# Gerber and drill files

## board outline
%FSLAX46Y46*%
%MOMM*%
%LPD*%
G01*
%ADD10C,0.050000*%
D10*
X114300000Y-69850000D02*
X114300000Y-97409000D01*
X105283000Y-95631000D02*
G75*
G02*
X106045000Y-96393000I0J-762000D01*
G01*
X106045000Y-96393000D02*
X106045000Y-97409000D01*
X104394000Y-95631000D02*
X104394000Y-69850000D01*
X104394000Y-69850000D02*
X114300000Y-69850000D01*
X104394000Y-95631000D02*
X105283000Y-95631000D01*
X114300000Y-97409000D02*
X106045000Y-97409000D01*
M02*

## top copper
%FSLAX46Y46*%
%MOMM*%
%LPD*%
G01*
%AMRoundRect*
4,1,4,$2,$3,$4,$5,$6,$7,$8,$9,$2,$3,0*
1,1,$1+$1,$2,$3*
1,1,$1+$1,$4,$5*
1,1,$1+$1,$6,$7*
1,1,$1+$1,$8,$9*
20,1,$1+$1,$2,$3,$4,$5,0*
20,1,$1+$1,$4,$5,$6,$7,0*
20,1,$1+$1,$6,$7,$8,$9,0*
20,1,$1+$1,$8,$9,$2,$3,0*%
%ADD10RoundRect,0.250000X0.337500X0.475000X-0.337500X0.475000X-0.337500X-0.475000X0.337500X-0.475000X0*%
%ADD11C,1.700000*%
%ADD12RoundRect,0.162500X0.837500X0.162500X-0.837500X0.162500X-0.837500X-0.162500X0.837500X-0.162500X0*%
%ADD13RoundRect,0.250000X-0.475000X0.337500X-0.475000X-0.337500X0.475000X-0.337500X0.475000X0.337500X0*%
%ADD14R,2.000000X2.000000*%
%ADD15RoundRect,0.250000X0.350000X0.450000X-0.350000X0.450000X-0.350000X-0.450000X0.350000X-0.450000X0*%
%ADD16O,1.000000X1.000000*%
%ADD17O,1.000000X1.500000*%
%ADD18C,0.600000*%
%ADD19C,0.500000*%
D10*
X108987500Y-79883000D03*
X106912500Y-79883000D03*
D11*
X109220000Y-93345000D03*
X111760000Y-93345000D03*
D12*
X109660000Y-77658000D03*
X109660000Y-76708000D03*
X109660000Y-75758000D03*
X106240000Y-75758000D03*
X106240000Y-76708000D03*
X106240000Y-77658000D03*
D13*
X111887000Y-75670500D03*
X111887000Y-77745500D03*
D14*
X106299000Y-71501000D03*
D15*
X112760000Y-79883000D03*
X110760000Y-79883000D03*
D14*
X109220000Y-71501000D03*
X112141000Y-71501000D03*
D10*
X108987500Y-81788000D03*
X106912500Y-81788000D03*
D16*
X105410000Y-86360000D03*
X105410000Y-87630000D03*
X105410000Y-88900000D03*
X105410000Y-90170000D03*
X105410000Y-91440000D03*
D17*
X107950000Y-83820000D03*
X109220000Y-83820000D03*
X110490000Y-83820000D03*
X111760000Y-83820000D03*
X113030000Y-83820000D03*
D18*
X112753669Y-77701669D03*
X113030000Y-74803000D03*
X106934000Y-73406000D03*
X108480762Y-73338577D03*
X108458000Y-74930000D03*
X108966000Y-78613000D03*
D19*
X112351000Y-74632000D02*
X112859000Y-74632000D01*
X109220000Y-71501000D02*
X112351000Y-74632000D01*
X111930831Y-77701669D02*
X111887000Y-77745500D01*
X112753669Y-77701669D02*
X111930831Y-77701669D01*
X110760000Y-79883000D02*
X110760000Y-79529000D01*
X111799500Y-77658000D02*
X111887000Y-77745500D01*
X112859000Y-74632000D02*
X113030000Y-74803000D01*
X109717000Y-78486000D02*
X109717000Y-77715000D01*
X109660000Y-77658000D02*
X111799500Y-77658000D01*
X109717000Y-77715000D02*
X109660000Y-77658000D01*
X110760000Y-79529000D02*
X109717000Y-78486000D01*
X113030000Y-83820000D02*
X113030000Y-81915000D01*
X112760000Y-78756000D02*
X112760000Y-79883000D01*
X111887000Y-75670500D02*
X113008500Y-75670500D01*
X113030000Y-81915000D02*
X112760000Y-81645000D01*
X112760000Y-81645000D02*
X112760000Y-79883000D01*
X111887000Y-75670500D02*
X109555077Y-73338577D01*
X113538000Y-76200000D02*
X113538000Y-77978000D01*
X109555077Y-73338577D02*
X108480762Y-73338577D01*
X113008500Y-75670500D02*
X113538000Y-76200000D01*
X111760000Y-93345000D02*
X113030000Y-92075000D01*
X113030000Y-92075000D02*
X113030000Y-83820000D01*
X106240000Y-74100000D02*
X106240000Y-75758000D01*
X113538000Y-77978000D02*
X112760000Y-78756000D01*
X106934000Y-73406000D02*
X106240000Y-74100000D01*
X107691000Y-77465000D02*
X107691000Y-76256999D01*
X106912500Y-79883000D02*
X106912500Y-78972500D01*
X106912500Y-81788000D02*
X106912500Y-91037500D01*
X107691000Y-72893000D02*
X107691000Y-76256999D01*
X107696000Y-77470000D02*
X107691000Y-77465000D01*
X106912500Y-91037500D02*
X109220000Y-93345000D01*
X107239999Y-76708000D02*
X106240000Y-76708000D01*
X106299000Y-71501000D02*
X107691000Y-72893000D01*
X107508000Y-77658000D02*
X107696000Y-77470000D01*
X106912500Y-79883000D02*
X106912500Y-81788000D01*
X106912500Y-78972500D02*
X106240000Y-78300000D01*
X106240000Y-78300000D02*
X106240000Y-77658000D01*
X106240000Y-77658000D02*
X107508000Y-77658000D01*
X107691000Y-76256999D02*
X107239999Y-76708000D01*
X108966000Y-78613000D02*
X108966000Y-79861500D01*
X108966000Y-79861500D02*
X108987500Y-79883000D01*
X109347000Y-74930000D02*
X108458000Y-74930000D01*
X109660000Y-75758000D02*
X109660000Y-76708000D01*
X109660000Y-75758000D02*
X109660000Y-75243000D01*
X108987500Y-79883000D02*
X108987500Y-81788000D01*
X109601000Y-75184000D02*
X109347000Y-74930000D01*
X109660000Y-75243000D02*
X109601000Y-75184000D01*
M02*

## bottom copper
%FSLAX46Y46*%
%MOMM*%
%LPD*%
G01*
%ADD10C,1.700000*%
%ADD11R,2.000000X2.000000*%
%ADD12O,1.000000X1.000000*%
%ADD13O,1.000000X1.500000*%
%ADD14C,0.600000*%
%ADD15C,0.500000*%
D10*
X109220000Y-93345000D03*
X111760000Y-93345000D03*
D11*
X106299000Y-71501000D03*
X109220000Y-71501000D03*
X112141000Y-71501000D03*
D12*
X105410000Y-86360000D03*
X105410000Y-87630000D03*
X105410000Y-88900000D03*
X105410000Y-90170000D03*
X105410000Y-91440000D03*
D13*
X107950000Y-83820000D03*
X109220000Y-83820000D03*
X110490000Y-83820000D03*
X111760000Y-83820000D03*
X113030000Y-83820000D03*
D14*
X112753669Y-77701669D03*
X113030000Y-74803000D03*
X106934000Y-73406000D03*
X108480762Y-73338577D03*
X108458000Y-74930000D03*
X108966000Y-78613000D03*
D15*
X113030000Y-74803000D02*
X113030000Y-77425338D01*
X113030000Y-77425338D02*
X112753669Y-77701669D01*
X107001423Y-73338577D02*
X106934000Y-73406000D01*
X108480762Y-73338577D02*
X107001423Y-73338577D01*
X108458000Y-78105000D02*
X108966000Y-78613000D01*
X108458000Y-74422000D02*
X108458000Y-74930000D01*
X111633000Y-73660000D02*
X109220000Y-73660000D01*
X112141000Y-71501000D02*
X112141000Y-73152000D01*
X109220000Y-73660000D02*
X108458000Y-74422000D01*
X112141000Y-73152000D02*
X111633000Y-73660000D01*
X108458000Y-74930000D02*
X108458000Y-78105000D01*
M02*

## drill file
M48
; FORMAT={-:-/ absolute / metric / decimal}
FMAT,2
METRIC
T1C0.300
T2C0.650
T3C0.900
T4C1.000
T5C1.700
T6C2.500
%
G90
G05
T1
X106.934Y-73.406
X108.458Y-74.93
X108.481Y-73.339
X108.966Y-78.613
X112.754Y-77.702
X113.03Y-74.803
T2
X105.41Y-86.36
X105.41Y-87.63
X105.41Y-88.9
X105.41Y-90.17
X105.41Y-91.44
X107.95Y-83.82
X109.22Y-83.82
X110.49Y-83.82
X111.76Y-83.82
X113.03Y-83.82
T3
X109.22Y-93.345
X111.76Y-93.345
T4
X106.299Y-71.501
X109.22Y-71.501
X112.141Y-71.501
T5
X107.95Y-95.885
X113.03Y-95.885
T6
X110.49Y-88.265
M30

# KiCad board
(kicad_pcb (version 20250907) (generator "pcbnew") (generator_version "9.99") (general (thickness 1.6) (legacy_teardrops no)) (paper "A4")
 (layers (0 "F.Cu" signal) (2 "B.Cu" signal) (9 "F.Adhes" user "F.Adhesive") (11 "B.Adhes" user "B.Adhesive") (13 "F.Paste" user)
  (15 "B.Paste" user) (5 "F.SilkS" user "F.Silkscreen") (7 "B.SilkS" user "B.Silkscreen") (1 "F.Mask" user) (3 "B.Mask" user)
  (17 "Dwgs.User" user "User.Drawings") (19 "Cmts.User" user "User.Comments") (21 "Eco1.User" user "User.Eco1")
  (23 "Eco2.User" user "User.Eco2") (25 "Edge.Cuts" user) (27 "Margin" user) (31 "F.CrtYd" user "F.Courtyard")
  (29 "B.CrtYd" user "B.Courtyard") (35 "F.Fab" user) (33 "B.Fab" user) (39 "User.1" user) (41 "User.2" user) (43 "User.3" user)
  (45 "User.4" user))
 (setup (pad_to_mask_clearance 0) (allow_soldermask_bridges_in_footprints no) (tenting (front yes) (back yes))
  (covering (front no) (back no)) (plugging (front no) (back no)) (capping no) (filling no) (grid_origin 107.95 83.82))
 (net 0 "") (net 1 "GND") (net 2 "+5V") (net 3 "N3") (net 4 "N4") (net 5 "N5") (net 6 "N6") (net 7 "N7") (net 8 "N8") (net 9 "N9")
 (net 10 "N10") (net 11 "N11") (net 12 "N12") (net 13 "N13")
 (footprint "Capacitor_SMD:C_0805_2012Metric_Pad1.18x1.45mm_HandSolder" (layer "F.Cu") (at 107.95 79.883 180)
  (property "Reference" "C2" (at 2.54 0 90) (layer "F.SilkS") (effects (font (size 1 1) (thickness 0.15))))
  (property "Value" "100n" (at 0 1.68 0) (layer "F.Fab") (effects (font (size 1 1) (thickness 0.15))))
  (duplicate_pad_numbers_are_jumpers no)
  (pad "1" smd roundrect (at -1.0375 0 180) (size 1.175 1.45) (layers "F.Cu" "F.Mask" "F.Paste") (roundrect_rratio 0.212766) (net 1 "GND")
   (tenting (front none) (back none)))
  (pad "2" smd roundrect (at 1.0375 0 180) (size 1.175 1.45) (layers "F.Cu" "F.Mask" "F.Paste") (roundrect_rratio 0.212766) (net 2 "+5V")
   (tenting (front none) (back none))))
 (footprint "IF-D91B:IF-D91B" (layer "F.Cu") (at 110.49 88.265 180)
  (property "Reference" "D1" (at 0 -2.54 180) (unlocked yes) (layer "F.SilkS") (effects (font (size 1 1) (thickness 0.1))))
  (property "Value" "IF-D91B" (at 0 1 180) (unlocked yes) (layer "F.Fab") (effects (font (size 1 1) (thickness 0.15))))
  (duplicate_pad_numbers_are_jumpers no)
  (pad "" np_thru_hole circle (at -2.54 -7.62 180) (size 1.7 1.7) (drill 1.7) (layers "*.Cu" "*.Mask") (tenting (front none) (back none)))
  (pad "" np_thru_hole circle (at 0 0 180) (size 2.5 2.5) (drill 2.5) (layers "*.Cu" "*.Mask") (tenting (front none) (back none)))
  (pad "" np_thru_hole circle (at 2.54 -7.62 180) (size 1.7 1.7) (drill 1.7) (layers "*.Cu" "*.Mask") (tenting (front none) (back none)))
  (pad "1" thru_hole circle (at 1.27 -5.08 180) (size 1.7 1.7) (drill 0.9) (layers "*.Cu" "*.Mask") (remove_unused_layers no) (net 2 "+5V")
   (tenting (front none) (back none)))
  (pad "2" thru_hole circle (at -1.27 -5.08 180) (size 1.7 1.7) (drill 0.9) (layers "*.Cu" "*.Mask") (remove_unused_layers no) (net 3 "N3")
   (tenting (front none) (back none))))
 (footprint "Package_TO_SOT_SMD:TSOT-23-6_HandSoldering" (layer "F.Cu") (at 107.95 76.708 180)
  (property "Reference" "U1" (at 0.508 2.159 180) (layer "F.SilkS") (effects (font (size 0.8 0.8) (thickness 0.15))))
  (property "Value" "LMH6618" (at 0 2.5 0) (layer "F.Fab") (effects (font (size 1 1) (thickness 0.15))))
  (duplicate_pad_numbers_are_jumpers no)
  (pad "1" smd roundrect (at -1.71 -0.95 180) (size 2 0.65) (layers "F.Cu" "F.Mask" "F.Paste") (roundrect_rratio 0.25) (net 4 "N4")
   (tenting (front none) (back none)))
  (pad "2" smd roundrect (at -1.71 0 180) (size 2 0.65) (layers "F.Cu" "F.Mask" "F.Paste") (roundrect_rratio 0.25) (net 1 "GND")
   (tenting (front none) (back none)))
  (pad "3" smd roundrect (at -1.71 0.95 180) (size 2 0.65) (layers "F.Cu" "F.Mask" "F.Paste") (roundrect_rratio 0.25) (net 1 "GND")
   (tenting (front none) (back none)))
  (pad "4" smd roundrect (at 1.71 0.95 180) (size 2 0.65) (layers "F.Cu" "F.Mask" "F.Paste") (roundrect_rratio 0.25) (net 3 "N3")
   (tenting (front none) (back none)))
  (pad "5" smd roundrect (at 1.71 0 180) (size 2 0.65) (layers "F.Cu" "F.Mask" "F.Paste") (roundrect_rratio 0.25) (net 2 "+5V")
   (tenting (front none) (back none)))
  (pad "6" smd roundrect (at 1.71 -0.95 180) (size 2 0.65) (layers "F.Cu" "F.Mask" "F.Paste") (roundrect_rratio 0.25) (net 2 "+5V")
   (tenting (front none) (back none))))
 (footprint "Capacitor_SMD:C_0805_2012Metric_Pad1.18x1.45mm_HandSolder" (layer "F.Cu") (at 111.887 76.708 -90)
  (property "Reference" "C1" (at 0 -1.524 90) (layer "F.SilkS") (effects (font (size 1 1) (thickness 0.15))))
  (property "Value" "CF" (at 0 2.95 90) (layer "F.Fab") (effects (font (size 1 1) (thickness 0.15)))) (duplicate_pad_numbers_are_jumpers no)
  (pad "1" smd roundrect (at -1.0375 0 270) (size 1.175 1.45) (layers "F.Cu" "F.Mask" "F.Paste") (roundrect_rratio 0.212766) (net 3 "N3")
   (tenting (front none) (back none)))
  (pad "2" smd roundrect (at 1.0375 0 270) (size 1.175 1.45) (layers "F.Cu" "F.Mask" "F.Paste") (roundrect_rratio 0.212766) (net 4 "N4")
   (tenting (front none) (back none))))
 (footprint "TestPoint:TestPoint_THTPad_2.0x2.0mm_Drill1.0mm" (layer "F.Cu") (at 106.299 71.501)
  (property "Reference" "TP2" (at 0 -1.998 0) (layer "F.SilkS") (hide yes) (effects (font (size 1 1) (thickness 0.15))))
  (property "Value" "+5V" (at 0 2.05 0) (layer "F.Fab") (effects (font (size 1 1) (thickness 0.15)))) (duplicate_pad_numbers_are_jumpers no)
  (pad "1" thru_hole rect (at 0 0) (size 2 2) (drill 1) (layers "*.Cu" "*.Mask") (remove_unused_layers no) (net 2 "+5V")
   (tenting (front none) (back none))))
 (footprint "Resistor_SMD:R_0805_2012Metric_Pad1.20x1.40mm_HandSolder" (layer "F.Cu") (at 111.76 79.883 180)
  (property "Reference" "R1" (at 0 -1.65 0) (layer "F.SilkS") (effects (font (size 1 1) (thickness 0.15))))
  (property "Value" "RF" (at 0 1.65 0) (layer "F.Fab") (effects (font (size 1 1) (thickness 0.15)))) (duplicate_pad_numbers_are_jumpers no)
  (pad "1" smd roundrect (at -1 0 180) (size 1.2 1.4) (layers "F.Cu" "F.Mask" "F.Paste") (roundrect_rratio 0.208333) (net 3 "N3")
   (tenting (front none) (back none)))
  (pad "2" smd roundrect (at 1 0 180) (size 1.2 1.4) (layers "F.Cu" "F.Mask" "F.Paste") (roundrect_rratio 0.208333) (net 4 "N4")
   (tenting (front none) (back none))))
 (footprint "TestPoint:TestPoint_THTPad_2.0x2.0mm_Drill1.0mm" (layer "F.Cu") (at 109.22 71.501)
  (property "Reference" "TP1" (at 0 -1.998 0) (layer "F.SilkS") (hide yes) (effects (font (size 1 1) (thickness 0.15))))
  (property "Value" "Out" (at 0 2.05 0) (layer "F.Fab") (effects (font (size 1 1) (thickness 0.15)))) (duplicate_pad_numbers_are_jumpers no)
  (pad "1" thru_hole rect (at 0 0) (size 2 2) (drill 1) (layers "*.Cu" "*.Mask") (remove_unused_layers no) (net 4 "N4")
   (tenting (front none) (back none))))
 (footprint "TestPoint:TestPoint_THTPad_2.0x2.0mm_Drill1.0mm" (layer "F.Cu") (at 112.141 71.501)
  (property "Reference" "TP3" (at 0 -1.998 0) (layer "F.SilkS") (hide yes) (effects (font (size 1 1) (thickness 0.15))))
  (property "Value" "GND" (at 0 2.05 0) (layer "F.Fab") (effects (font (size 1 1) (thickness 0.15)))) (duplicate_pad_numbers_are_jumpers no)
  (pad "1" thru_hole rect (at 0 0) (size 2 2) (drill 1) (layers "*.Cu" "*.Mask") (remove_unused_layers no) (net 1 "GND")
   (tenting (front none) (back none))))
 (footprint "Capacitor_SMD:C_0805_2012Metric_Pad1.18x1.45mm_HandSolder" (layer "F.Cu") (at 107.95 81.788 180)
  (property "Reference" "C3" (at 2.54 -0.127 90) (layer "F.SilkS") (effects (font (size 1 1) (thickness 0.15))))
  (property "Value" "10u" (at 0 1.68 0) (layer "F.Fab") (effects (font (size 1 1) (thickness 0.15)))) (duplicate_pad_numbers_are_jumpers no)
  (pad "1" smd roundrect (at -1.0375 0 180) (size 1.175 1.45) (layers "F.Cu" "F.Mask" "F.Paste") (roundrect_rratio 0.212766) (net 1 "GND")
   (tenting (front none) (back none)))
  (pad "2" smd roundrect (at 1.0375 0 180) (size 1.175 1.45) (layers "F.Cu" "F.Mask" "F.Paste") (roundrect_rratio 0.212766) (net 2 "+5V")
   (tenting (front none) (back none))))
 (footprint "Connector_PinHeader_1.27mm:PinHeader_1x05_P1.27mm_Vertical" (layer "B.Cu") (at 105.41 86.36 180)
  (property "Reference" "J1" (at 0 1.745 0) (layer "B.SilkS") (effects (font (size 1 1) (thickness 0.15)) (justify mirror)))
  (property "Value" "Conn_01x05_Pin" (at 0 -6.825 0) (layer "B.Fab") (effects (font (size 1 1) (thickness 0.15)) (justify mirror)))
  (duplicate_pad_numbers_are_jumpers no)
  (pad "1" thru_hole oval (at 0 0 180) (size 1 1) (drill 0.65) (layers "*.Cu" "*.Mask") (remove_unused_layers no) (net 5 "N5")
   (tenting (front none) (back none)))
  (pad "2" thru_hole oval (at 0 -1.27 180) (size 1 1) (drill 0.65) (layers "*.Cu" "*.Mask") (remove_unused_layers no) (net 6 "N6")
   (thermal_bridge_angle 45) (tenting (front none) (back none)))
  (pad "3" thru_hole oval (at 0 -2.54 180) (size 1 1) (drill 0.65) (layers "*.Cu" "*.Mask") (remove_unused_layers no) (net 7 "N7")
   (thermal_bridge_angle 45) (tenting (front none) (back none)))
  (pad "4" thru_hole oval (at 0 -3.81 180) (size 1 1) (drill 0.65) (layers "*.Cu" "*.Mask") (remove_unused_layers no) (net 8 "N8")
   (thermal_bridge_angle 45) (tenting (front none) (back none)))
  (pad "5" thru_hole oval (at 0 -5.08 180) (size 1 1) (drill 0.65) (layers "*.Cu" "*.Mask") (remove_unused_layers no) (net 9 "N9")
   (thermal_bridge_angle 45) (tenting (front none) (back none))))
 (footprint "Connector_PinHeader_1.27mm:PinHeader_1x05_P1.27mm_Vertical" (layer "B.Cu") (at 107.95 83.82 -90)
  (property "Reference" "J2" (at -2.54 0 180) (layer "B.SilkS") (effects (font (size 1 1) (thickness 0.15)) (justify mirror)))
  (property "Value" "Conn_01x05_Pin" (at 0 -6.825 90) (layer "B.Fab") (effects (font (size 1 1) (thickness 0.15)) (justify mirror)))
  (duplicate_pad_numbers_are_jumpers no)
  (pad "1" thru_hole oval (at 0 0 270) (size 1.5 1) (drill 0.65) (layers "*.Cu" "*.Mask") (remove_unused_layers no) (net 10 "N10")
   (tenting (front none) (back none)))
  (pad "2" thru_hole oval (at 0 -1.27 270) (size 1.5 1) (drill 0.65) (layers "*.Cu" "*.Mask") (remove_unused_layers no) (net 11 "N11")
   (thermal_bridge_angle 45) (tenting (front none) (back none)))
  (pad "3" thru_hole oval (at 0 -2.54 270) (size 1.5 1) (drill 0.65) (layers "*.Cu" "*.Mask") (remove_unused_layers no) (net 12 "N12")
   (thermal_bridge_angle 45) (tenting (front none) (back none)))
  (pad "4" thru_hole oval (at 0 -3.81 270) (size 1.5 1) (drill 0.65) (layers "*.Cu" "*.Mask") (remove_unused_layers no) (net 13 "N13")
   (thermal_bridge_angle 45) (tenting (front none) (back none)))
  (pad "5" thru_hole oval (at 0 -5.08 270) (size 1.5 1) (drill 0.65) (layers "*.Cu" "*.Mask") (remove_unused_layers no) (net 3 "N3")
   (thermal_bridge_angle 45) (tenting (front none) (back none))))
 (gr_line (start 114.3 69.85) (end 114.3 97.409) (stroke (width 0.05) (type default)) (layer "Edge.Cuts"))
 (gr_arc (start 105.283 95.631) (mid 105.821815 95.854185) (end 106.045 96.393) (stroke (width 0.05) (type default)) (layer "Edge.Cuts"))
 (gr_line (start 106.045 96.393) (end 106.045 97.409) (stroke (width 0.05) (type default)) (layer "Edge.Cuts"))
 (gr_line (start 104.394 95.631) (end 104.394 69.85) (stroke (width 0.05) (type default)) (layer "Edge.Cuts"))
 (gr_line (start 104.394 69.85) (end 114.3 69.85) (stroke (width 0.05) (type default)) (layer "Edge.Cuts"))
 (gr_line (start 104.394 95.631) (end 105.283 95.631) (stroke (width 0.05) (type default)) (layer "Edge.Cuts"))
 (gr_line (start 114.3 97.409) (end 106.045 97.409) (stroke (width 0.05) (type default)) (layer "Edge.Cuts"))
 (segment (start 112.351 74.632) (end 112.859 74.632) (width 0.5) (layer "F.Cu") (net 4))
 (segment (start 109.22 71.501) (end 112.351 74.632) (width 0.5) (layer "F.Cu") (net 4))
 (segment (start 111.930831 77.701669) (end 111.887 77.7455) (width 0.5) (layer "F.Cu") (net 4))
 (segment (start 112.753669 77.701669) (end 111.930831 77.701669) (width 0.5) (layer "F.Cu") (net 4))
 (segment (start 110.76 79.883) (end 110.76 79.529) (width 0.5) (layer "F.Cu") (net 4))
 (segment (start 111.7995 77.658) (end 111.887 77.7455) (width 0.5) (layer "F.Cu") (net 4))
 (segment (start 112.859 74.632) (end 113.03 74.803) (width 0.5) (layer "F.Cu") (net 4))
 (segment (start 109.717 78.486) (end 109.717 77.715) (width 0.5) (layer "F.Cu") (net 4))
 (segment (start 109.66 77.658) (end 111.7995 77.658) (width 0.5) (layer "F.Cu") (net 4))
 (segment (start 109.717 77.715) (end 109.66 77.658) (width 0.5) (layer "F.Cu") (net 4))
 (segment (start 110.76 79.529) (end 109.717 78.486) (width 0.5) (layer "F.Cu") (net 4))
 (via (at 112.753669 77.701669) (size 0.6) (drill 0.3) (layers "F.Cu" "B.Cu") (tenting (front none) (back none)) (capping none)
  (covering (front none) (back none)) (plugging (front none) (back none)) (filling none) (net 4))
 (via (at 113.03 74.803) (size 0.6) (drill 0.3) (layers "F.Cu" "B.Cu") (tenting (front none) (back none)) (capping none)
  (covering (front none) (back none)) (plugging (front none) (back none)) (filling none) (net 4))
 (segment (start 113.03 74.803) (end 113.03 77.425338) (width 0.5) (layer "B.Cu") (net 4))
 (segment (start 113.03 77.425338) (end 112.753669 77.701669) (width 0.5) (layer "B.Cu") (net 4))
 (segment (start 113.03 83.82) (end 113.03 81.915) (width 0.5) (layer "F.Cu") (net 3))
 (segment (start 112.76 78.756) (end 112.76 79.883) (width 0.5) (layer "F.Cu") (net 3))
 (segment (start 111.887 75.6705) (end 113.0085 75.6705) (width 0.5) (layer "F.Cu") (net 3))
 (segment (start 113.03 81.915) (end 112.76 81.645) (width 0.5) (layer "F.Cu") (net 3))
 (segment (start 112.76 81.645) (end 112.76 79.883) (width 0.5) (layer "F.Cu") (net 3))
 (segment (start 111.887 75.6705) (end 109.555077 73.338577) (width 0.5) (layer "F.Cu") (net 3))
 (segment (start 113.538 76.2) (end 113.538 77.978) (width 0.5) (layer "F.Cu") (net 3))
 (segment (start 109.555077 73.338577) (end 108.480762 73.338577) (width 0.5) (layer "F.Cu") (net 3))
 (segment (start 113.0085 75.6705) (end 113.538 76.2) (width 0.5) (layer "F.Cu") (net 3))
 (segment (start 111.76 93.345) (end 113.03 92.075) (width 0.5) (layer "F.Cu") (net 3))
 (segment (start 113.03 92.075) (end 113.03 83.82) (width 0.5) (layer "F.Cu") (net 3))
 (segment (start 106.24 74.1) (end 106.24 75.758) (width 0.5) (layer "F.Cu") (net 3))
 (segment (start 113.538 77.978) (end 112.76 78.756) (width 0.5) (layer "F.Cu") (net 3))
 (segment (start 106.934 73.406) (end 106.24 74.1) (width 0.5) (layer "F.Cu") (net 3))
 (via (at 106.934 73.406) (size 0.6) (drill 0.3) (layers "F.Cu" "B.Cu") (tenting (front none) (back none)) (capping none)
  (covering (front none) (back none)) (plugging (front none) (back none)) (filling none) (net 3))
 (via (at 108.480762 73.338577) (size 0.6) (drill 0.3) (layers "F.Cu" "B.Cu") (tenting (front none) (back none)) (capping none)
  (covering (front none) (back none)) (plugging (front none) (back none)) (filling none) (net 3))
 (segment (start 107.001423 73.338577) (end 106.934 73.406) (width 0.5) (layer "B.Cu") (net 3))
 (segment (start 108.480762 73.338577) (end 107.001423 73.338577) (width 0.5) (layer "B.Cu") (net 3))
 (segment (start 107.691 77.465) (end 107.691 76.256999) (width 0.5) (layer "F.Cu") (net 2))
 (segment (start 106.9125 79.883) (end 106.9125 78.9725) (width 0.5) (layer "F.Cu") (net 2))
 (segment (start 106.9125 81.788) (end 106.9125 91.0375) (width 0.5) (layer "F.Cu") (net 2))
 (segment (start 107.691 72.893) (end 107.691 76.256999) (width 0.5) (layer "F.Cu") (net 2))
 (segment (start 107.696 77.47) (end 107.691 77.465) (width 0.5) (layer "F.Cu") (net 2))
 (segment (start 106.9125 91.0375) (end 109.22 93.345) (width 0.5) (layer "F.Cu") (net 2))
 (segment (start 107.239999 76.708) (end 106.24 76.708) (width 0.5) (layer "F.Cu") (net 2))
 (segment (start 106.299 71.501) (end 107.691 72.893) (width 0.5) (layer "F.Cu") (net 2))
 (segment (start 107.508 77.658) (end 107.696 77.47) (width 0.5) (layer "F.Cu") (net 2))
 (segment (start 106.9125 79.883) (end 106.9125 81.788) (width 0.5) (layer "F.Cu") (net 2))
 (segment (start 106.9125 78.9725) (end 106.24 78.3) (width 0.5) (layer "F.Cu") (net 2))
 (segment (start 106.24 78.3) (end 106.24 77.658) (width 0.5) (layer "F.Cu") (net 2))
 (segment (start 106.24 77.658) (end 107.508 77.658) (width 0.5) (layer "F.Cu") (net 2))
 (segment (start 107.691 76.256999) (end 107.239999 76.708) (width 0.5) (layer "F.Cu") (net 2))
 (segment (start 108.966 78.613) (end 108.966 79.8615) (width 0.5) (layer "F.Cu") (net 1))
 (segment (start 108.966 79.8615) (end 108.9875 79.883) (width 0.5) (layer "F.Cu") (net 1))
 (segment (start 109.347 74.93) (end 108.458 74.93) (width 0.5) (layer "F.Cu") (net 1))
 (segment (start 109.66 75.758) (end 109.66 76.708) (width 0.5) (layer "F.Cu") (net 1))
 (segment (start 109.66 75.758) (end 109.66 75.243) (width 0.5) (layer "F.Cu") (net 1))
 (segment (start 108.9875 79.883) (end 108.9875 81.788) (width 0.5) (layer "F.Cu") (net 1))
 (segment (start 109.601 75.184) (end 109.347 74.93) (width 0.5) (layer "F.Cu") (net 1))
 (segment (start 109.66 75.243) (end 109.601 75.184) (width 0.5) (layer "F.Cu") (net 1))
 (via (at 108.458 74.93) (size 0.6) (drill 0.3) (layers "F.Cu" "B.Cu") (tenting (front none) (back none)) (capping none)
  (covering (front none) (back none)) (plugging (front none) (back none)) (filling none) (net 1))
 (via (at 108.966 78.613) (size 0.6) (drill 0.3) (layers "F.Cu" "B.Cu") (tenting (front none) (back none)) (capping none)
  (covering (front none) (back none)) (plugging (front none) (back none)) (filling none) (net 1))
 (segment (start 108.458 78.105) (end 108.966 78.613) (width 0.5) (layer "B.Cu") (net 1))
 (segment (start 108.458 74.422) (end 108.458 74.93) (width 0.5) (layer "B.Cu") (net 1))
 (segment (start 111.633 73.66) (end 109.22 73.66) (width 0.5) (layer "B.Cu") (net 1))
 (segment (start 112.141 71.501) (end 112.141 73.152) (width 0.5) (layer "B.Cu") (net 1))
 (segment (start 109.22 73.66) (end 108.458 74.422) (width 0.5) (layer "B.Cu") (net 1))
 (segment (start 112.141 73.152) (end 111.633 73.66) (width 0.5) (layer "B.Cu") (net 1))
 (segment (start 108.458 74.93) (end 108.458 78.105) (width 0.5) (layer "B.Cu") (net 1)))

